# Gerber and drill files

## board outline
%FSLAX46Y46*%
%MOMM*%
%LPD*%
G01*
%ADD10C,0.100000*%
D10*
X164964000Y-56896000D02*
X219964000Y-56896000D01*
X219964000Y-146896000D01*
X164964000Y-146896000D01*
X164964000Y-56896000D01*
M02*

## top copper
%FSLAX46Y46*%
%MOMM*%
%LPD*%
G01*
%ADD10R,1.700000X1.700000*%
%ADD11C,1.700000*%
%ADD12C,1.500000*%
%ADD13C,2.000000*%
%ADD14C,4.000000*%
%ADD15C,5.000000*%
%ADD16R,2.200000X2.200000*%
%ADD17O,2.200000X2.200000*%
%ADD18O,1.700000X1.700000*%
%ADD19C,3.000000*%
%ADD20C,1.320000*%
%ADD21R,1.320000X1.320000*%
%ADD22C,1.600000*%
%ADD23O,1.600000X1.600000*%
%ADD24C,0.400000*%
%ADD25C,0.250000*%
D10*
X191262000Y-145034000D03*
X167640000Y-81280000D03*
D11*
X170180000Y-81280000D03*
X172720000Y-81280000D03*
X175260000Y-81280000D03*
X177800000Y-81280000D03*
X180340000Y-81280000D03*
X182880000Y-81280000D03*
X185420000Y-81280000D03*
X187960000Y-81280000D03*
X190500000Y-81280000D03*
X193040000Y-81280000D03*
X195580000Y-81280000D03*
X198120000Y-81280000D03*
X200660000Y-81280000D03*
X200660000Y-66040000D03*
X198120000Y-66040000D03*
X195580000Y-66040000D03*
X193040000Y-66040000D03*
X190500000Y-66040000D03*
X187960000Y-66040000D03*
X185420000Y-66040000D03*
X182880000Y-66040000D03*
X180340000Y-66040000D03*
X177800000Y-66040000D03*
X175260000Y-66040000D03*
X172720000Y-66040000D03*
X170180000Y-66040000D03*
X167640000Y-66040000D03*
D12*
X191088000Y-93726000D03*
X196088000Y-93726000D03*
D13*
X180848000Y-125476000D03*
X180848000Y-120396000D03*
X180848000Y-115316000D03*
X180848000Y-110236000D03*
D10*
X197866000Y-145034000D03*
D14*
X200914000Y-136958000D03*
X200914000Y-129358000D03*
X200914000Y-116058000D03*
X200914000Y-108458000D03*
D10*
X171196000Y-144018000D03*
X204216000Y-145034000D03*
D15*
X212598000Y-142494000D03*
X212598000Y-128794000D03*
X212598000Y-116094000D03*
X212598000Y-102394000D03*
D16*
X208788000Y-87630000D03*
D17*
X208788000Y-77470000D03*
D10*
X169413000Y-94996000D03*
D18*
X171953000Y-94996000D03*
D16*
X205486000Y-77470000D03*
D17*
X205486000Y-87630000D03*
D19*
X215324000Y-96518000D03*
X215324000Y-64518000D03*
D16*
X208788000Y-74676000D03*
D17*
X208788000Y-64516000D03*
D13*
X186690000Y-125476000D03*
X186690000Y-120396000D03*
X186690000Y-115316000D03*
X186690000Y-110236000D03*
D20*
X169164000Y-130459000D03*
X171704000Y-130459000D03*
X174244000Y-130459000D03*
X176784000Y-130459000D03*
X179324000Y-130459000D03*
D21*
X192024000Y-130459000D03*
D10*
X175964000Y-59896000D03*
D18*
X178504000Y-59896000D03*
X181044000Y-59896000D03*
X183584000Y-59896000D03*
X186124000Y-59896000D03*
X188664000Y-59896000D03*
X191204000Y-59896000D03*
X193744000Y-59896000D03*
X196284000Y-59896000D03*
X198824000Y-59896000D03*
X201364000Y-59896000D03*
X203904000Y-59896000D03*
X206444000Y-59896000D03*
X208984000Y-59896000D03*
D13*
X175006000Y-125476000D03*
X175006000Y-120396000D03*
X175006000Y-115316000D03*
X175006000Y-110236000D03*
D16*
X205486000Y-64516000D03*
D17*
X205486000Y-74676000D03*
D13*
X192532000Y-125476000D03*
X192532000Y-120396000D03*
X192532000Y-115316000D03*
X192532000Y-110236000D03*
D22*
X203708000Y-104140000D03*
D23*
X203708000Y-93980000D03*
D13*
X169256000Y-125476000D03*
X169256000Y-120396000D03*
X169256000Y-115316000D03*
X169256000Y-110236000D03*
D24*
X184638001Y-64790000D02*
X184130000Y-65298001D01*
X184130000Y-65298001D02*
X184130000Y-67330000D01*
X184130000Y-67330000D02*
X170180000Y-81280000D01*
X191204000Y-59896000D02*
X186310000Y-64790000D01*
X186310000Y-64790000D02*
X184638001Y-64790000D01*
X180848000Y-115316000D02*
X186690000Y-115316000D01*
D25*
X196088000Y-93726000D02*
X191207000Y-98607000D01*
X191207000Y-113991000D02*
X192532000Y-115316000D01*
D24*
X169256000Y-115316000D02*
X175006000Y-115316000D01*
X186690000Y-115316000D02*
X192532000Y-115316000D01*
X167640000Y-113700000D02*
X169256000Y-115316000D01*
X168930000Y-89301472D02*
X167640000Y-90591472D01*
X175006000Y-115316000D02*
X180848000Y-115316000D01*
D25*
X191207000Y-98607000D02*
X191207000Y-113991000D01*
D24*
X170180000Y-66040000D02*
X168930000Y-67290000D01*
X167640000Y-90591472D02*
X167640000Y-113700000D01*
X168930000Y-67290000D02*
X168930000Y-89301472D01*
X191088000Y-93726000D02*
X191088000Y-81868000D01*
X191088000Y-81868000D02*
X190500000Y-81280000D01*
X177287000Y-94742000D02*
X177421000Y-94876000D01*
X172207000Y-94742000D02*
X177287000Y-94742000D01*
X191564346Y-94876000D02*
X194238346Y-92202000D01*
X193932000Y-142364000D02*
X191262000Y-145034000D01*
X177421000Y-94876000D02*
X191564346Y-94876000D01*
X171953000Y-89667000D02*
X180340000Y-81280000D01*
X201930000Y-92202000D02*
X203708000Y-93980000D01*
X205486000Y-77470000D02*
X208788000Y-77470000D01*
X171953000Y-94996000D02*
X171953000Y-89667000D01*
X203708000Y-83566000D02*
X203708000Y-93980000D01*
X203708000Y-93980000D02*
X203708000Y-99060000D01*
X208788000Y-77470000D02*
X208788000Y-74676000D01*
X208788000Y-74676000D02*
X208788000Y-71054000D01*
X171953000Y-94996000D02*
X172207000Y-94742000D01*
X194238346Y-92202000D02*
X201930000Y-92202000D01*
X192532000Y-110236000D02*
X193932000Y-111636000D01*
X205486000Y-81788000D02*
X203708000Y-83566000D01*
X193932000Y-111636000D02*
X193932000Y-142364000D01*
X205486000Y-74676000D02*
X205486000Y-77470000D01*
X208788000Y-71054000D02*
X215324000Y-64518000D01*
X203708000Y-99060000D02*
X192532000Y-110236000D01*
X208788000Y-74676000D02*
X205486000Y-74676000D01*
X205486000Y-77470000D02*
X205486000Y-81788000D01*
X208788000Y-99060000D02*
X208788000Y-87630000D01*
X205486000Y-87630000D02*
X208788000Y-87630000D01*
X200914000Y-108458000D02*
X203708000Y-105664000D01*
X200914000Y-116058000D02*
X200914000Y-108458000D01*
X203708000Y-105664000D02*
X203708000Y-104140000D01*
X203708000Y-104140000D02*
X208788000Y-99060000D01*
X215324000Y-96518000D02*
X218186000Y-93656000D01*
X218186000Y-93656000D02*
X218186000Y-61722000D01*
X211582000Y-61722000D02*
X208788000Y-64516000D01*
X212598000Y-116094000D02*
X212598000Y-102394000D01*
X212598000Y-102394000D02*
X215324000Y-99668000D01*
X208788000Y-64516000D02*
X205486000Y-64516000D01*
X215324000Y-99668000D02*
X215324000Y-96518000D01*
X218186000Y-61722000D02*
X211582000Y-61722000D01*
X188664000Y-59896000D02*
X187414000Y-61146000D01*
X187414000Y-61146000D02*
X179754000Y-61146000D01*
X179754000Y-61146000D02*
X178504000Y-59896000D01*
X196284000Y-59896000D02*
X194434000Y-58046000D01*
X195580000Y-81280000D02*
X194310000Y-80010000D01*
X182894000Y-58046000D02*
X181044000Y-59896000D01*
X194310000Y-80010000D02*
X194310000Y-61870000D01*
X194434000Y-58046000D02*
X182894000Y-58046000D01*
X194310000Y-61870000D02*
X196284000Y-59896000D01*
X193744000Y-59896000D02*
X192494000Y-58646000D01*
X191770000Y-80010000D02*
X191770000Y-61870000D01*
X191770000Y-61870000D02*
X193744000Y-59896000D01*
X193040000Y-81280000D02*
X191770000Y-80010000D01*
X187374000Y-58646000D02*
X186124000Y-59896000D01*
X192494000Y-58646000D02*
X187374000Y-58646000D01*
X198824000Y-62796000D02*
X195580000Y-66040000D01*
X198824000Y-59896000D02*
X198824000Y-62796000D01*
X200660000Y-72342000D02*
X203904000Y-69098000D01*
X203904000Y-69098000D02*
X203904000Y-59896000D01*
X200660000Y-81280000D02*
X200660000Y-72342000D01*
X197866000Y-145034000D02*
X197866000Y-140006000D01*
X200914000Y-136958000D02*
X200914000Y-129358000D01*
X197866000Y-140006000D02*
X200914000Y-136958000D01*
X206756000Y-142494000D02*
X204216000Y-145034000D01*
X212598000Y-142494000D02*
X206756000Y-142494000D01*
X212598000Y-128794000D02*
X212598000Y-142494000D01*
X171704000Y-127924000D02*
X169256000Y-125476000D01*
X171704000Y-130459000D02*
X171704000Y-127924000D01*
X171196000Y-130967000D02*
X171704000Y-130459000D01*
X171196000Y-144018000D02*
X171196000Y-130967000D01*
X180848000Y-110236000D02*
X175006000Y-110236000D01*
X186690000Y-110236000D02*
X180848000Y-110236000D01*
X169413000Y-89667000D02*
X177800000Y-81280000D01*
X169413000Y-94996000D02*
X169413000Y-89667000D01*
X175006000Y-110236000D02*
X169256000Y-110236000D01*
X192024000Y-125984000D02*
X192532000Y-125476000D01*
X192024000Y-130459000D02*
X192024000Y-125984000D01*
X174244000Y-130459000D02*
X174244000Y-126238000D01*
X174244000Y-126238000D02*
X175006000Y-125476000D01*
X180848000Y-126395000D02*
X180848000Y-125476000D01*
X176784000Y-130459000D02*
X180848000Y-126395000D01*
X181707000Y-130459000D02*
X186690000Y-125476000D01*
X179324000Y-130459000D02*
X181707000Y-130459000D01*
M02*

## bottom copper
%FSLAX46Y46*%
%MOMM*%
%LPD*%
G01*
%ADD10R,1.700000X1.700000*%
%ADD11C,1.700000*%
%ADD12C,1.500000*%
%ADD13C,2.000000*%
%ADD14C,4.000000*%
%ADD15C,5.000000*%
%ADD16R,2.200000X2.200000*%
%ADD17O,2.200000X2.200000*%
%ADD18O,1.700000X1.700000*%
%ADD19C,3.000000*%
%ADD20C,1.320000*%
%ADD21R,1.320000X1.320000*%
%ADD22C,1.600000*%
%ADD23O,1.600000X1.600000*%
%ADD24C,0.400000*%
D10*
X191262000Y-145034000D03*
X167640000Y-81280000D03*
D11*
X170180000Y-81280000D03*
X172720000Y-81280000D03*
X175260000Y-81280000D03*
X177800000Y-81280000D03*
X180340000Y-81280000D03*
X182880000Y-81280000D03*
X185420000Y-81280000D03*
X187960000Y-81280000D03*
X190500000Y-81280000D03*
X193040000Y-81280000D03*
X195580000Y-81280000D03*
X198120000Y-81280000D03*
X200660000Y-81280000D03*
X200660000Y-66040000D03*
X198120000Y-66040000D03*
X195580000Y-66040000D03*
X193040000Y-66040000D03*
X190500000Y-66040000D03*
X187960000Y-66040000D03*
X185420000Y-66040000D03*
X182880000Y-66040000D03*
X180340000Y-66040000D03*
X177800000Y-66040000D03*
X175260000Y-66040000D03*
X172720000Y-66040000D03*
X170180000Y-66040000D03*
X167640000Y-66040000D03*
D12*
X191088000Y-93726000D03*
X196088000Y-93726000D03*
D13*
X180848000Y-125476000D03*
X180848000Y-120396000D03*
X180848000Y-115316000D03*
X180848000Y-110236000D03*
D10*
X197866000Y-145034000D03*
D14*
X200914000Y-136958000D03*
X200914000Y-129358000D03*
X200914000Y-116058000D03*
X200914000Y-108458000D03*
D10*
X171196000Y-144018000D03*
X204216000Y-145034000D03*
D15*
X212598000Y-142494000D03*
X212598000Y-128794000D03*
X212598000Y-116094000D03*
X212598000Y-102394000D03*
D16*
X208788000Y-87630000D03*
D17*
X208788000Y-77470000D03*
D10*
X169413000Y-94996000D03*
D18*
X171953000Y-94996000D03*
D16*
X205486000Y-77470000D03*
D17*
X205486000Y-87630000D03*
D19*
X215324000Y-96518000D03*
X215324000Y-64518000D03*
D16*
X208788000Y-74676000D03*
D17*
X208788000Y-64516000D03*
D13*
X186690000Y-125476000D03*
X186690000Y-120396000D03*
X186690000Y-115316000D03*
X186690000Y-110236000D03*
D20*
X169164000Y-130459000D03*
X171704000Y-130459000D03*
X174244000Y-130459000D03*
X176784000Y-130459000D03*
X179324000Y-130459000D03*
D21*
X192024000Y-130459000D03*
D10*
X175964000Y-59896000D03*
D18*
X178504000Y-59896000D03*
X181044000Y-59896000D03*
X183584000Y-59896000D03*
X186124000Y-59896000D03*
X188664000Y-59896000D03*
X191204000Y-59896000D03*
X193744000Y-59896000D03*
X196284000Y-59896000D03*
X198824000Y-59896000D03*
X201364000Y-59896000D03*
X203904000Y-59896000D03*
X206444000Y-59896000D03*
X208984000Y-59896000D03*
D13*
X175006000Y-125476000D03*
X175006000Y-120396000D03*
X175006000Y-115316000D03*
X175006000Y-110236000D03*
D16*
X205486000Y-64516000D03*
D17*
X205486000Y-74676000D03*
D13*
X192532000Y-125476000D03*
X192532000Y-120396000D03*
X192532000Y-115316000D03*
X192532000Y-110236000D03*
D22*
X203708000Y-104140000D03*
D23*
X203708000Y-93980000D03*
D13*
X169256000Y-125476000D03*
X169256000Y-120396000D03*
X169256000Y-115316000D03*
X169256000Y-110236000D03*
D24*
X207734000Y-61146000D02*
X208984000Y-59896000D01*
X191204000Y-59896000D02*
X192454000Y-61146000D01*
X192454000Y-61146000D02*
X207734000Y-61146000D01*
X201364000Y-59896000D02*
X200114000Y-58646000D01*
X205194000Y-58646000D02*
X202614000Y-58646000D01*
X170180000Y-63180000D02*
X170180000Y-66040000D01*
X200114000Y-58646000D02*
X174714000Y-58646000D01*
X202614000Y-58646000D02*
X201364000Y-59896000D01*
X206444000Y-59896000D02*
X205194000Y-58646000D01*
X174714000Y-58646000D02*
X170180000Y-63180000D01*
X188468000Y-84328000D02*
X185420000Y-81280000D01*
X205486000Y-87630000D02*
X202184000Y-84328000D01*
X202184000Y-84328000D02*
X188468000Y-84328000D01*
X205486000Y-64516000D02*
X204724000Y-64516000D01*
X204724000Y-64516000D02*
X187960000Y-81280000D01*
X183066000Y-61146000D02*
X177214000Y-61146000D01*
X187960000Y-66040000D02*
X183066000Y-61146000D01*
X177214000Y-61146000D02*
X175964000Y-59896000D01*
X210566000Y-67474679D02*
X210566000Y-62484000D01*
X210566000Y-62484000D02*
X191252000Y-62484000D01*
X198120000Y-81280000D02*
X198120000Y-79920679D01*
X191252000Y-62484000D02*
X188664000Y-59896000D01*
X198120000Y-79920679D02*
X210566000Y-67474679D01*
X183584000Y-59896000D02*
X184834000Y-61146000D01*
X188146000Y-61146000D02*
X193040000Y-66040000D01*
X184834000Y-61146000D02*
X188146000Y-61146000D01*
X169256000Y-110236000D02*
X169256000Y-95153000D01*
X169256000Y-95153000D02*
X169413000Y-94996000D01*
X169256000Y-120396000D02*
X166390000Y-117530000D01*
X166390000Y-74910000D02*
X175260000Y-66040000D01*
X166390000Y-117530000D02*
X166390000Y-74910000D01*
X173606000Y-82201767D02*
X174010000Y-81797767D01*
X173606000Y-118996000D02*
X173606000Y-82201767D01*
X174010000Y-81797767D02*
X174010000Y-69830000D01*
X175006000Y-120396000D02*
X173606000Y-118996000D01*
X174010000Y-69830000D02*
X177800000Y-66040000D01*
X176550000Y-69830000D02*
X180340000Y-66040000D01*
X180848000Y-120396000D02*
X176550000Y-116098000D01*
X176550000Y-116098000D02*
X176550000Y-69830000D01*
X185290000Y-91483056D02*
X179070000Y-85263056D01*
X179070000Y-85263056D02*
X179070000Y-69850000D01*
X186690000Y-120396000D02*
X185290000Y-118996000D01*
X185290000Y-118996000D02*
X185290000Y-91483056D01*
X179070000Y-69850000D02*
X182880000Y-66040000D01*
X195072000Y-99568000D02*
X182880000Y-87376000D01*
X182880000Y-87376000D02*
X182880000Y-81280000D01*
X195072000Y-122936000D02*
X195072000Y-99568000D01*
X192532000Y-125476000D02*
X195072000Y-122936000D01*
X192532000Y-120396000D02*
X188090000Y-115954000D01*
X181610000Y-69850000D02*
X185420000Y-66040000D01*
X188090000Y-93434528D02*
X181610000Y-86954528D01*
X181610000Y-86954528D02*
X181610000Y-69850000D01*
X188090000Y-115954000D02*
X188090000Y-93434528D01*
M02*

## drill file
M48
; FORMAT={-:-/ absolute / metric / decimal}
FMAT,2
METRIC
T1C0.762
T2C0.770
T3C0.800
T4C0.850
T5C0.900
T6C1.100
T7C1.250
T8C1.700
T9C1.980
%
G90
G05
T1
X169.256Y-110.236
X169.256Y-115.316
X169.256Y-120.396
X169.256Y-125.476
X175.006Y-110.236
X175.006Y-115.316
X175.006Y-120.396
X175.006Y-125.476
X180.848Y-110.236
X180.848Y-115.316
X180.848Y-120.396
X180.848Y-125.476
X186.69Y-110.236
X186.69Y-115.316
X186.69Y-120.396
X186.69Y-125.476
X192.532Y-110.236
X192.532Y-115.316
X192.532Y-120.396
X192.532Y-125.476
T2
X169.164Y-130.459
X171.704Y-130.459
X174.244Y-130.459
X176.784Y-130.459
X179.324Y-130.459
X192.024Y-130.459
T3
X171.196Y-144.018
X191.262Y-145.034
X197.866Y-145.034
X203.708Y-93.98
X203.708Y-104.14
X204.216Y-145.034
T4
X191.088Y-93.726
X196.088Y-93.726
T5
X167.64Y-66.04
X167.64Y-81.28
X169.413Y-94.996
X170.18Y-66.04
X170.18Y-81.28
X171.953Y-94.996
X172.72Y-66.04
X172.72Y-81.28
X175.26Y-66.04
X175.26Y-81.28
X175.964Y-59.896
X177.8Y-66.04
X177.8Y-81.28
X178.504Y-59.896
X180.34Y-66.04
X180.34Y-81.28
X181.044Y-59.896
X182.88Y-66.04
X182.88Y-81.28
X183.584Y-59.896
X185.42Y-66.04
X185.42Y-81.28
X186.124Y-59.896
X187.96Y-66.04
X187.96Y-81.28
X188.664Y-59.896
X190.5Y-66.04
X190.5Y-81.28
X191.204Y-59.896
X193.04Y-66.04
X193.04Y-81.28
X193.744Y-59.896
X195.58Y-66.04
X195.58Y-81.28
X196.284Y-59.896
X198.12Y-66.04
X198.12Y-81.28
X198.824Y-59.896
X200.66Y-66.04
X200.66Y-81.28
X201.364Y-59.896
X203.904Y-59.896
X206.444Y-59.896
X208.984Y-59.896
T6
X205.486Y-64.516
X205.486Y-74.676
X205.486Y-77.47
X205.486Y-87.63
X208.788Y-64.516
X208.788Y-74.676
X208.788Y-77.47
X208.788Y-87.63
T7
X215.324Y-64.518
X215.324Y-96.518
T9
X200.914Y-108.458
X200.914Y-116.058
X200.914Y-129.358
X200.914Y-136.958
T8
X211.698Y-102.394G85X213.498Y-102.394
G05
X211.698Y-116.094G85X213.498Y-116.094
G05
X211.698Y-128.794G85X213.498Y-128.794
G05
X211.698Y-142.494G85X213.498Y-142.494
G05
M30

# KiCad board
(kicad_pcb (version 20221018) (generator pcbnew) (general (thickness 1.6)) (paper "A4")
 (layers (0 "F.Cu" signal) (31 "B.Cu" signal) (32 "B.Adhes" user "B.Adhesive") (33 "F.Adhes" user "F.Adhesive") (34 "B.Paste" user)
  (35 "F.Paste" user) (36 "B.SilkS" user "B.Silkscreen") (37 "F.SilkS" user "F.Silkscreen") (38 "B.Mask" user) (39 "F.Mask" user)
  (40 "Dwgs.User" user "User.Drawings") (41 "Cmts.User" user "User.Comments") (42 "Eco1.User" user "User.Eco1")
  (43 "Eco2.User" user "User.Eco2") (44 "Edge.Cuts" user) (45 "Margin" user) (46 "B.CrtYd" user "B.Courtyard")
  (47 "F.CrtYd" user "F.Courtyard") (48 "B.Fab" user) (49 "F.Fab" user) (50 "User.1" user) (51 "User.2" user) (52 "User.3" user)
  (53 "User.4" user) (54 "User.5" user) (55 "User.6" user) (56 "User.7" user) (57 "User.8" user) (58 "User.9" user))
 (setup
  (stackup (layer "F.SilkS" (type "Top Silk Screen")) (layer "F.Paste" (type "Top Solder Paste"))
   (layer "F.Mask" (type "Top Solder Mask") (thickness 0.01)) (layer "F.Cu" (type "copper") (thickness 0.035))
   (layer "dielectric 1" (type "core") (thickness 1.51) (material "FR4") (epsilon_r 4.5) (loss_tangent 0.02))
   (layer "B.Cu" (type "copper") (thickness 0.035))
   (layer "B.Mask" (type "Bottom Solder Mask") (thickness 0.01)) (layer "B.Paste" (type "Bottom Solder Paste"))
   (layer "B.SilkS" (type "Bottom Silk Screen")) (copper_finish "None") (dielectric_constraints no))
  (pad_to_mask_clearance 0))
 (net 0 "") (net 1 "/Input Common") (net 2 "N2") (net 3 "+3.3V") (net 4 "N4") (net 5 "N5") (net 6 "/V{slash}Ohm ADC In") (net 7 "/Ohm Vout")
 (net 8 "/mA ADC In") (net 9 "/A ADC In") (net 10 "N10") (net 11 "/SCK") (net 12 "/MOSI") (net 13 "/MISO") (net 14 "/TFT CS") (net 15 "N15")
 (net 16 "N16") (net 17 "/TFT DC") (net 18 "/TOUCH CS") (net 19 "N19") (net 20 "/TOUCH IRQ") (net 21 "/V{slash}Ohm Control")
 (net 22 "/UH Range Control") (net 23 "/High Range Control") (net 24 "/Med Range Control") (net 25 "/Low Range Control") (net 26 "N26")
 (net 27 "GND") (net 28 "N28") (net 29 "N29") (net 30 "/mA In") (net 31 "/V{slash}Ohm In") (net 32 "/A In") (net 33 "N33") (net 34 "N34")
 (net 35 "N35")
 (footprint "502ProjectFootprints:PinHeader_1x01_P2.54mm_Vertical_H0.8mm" (layer "F.Cu") (at 191.262 145.034)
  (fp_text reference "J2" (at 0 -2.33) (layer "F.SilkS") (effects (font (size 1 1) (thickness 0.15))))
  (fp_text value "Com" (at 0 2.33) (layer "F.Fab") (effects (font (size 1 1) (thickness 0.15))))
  (pad "1" thru_hole rect (at 0 0) (size 1.7 1.7) (drill 0.8) (layers "*.Cu" "*.Mask") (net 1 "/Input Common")))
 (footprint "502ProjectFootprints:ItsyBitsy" (layer "F.Cu") (at 182.88 73.66 90)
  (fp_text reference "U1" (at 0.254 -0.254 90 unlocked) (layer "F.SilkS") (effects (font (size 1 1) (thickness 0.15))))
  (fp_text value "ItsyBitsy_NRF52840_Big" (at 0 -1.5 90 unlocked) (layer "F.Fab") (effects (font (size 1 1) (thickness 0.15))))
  (pad "1" thru_hole rect (at -7.62 -15.24 90) (size 1.7 1.7) (drill 0.9) (layers "*.Cu" "*.Mask") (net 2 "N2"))
  (pad "2" thru_hole circle (at -7.62 -12.7 90) (size 1.7 1.7) (drill 0.9) (layers "*.Cu" "*.Mask") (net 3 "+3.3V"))
  (pad "3" thru_hole circle (at -7.62 -10.16 90) (size 1.7 1.7) (drill 0.9) (layers "*.Cu" "*.Mask") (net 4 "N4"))
  (pad "4" thru_hole circle (at -7.62 -7.62 90) (size 1.7 1.7) (drill 0.9) (layers "*.Cu" "*.Mask") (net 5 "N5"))
  (pad "5" thru_hole circle (at -7.62 -5.08 90) (size 1.7 1.7) (drill 0.9) (layers "*.Cu" "*.Mask") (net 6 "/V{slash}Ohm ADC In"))
  (pad "6" thru_hole circle (at -7.62 -2.54 90) (size 1.7 1.7) (drill 0.9) (layers "*.Cu" "*.Mask") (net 1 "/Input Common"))
  (pad "7" thru_hole circle (at -7.62 0 90) (size 1.7 1.7) (drill 0.9) (layers "*.Cu" "*.Mask") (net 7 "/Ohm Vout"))
  (pad "8" thru_hole circle (at -7.62 2.54 90) (size 1.7 1.7) (drill 0.9) (layers "*.Cu" "*.Mask") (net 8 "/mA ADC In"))
  (pad "9" thru_hole circle (at -7.62 5.08 90) (size 1.7 1.7) (drill 0.9) (layers "*.Cu" "*.Mask") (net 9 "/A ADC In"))
  (pad "10" thru_hole circle (at -7.62 7.62 90) (size 1.7 1.7) (drill 0.9) (layers "*.Cu" "*.Mask") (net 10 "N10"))
  (pad "11" thru_hole circle (at -7.62 10.16 90) (size 1.7 1.7) (drill 0.9) (layers "*.Cu" "*.Mask") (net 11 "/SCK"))
  (pad "12" thru_hole circle (at -7.62 12.7 90) (size 1.7 1.7) (drill 0.9) (layers "*.Cu" "*.Mask") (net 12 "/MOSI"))
  (pad "13" thru_hole circle (at -7.62 15.24 90) (size 1.7 1.7) (drill 0.9) (layers "*.Cu" "*.Mask") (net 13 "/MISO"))
  (pad "14" thru_hole circle (at -7.62 17.78 90) (size 1.7 1.7) (drill 0.9) (layers "*.Cu" "*.Mask") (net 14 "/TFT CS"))
  (pad "15" thru_hole circle (at 7.62 17.78 90) (size 1.7 1.7) (drill 0.9) (layers "*.Cu" "*.Mask") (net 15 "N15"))
  (pad "16" thru_hole circle (at 7.62 15.24 90) (size 1.7 1.7) (drill 0.9) (layers "*.Cu" "*.Mask") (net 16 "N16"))
  (pad "17" thru_hole circle (at 7.62 12.7 90) (size 1.7 1.7) (drill 0.9) (layers "*.Cu" "*.Mask") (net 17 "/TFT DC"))
  (pad "18" thru_hole circle (at 7.62 10.16 90) (size 1.7 1.7) (drill 0.9) (layers "*.Cu" "*.Mask") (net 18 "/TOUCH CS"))
  (pad "19" thru_hole circle (at 7.62 7.62 90) (size 1.7 1.7) (drill 0.9) (layers "*.Cu" "*.Mask") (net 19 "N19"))
  (pad "20" thru_hole circle (at 7.62 5.08 90) (size 1.7 1.7) (drill 0.9) (layers "*.Cu" "*.Mask") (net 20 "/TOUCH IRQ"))
  (pad "21" thru_hole circle (at 7.62 2.54 90) (size 1.7 1.7) (drill 0.9) (layers "*.Cu" "*.Mask") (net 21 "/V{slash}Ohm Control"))
  (pad "22" thru_hole circle (at 7.62 0 90) (size 1.7 1.7) (drill 0.9) (layers "*.Cu" "*.Mask") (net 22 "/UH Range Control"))
  (pad "23" thru_hole circle (at 7.62 -2.54 90) (size 1.7 1.7) (drill 0.9) (layers "*.Cu" "*.Mask") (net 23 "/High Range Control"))
  (pad "24" thru_hole circle (at 7.62 -5.08 90) (size 1.7 1.7) (drill 0.9) (layers "*.Cu" "*.Mask") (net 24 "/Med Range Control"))
  (pad "25" thru_hole circle (at 7.62 -7.62 90) (size 1.7 1.7) (drill 0.9) (layers "*.Cu" "*.Mask") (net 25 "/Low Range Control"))
  (pad "26" thru_hole circle (at 7.62 -10.16 90) (size 1.7 1.7) (drill 0.9) (layers "*.Cu" "*.Mask") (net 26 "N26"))
  (pad "27" thru_hole circle (at 7.62 -12.7 90) (size 1.7 1.7) (drill 0.9) (layers "*.Cu" "*.Mask") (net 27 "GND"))
  (pad "28" thru_hole circle (at 7.62 -15.24 90) (size 1.7 1.7) (drill 0.9) (layers "*.Cu" "*.Mask") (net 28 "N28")))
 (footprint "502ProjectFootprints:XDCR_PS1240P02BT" (layer "F.Cu") (at 193.588 93.726)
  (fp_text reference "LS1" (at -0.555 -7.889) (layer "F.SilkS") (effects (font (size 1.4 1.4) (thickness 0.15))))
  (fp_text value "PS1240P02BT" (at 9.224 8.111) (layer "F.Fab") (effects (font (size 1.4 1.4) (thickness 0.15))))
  (pad "1" thru_hole circle (at -2.5 0) (size 1.5 1.5) (drill 0.85) (layers "*.Cu" "*.Mask") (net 10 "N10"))
  (pad "2" thru_hole circle (at 2.5 0) (size 1.5 1.5) (drill 0.85) (layers "*.Cu" "*.Mask") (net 27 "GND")))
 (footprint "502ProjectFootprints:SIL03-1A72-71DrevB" (layer "F.Cu") (at 180.848 117.856 90)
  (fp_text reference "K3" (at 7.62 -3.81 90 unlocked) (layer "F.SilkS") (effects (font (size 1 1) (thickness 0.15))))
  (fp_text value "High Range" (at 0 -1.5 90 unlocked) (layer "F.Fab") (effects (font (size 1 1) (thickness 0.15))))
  (pad "1" thru_hole circle (at -7.62 0 90) (size 2 2) (drill 0.762) (layers "*.Cu" "*.Mask") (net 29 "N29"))
  (pad "3" thru_hole circle (at -2.54 0 90) (size 2 2) (drill 0.762) (layers "*.Cu" "*.Mask") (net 23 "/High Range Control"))
  (pad "5" thru_hole circle (at 2.54 0 90) (size 2 2) (drill 0.762) (layers "*.Cu" "*.Mask") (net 27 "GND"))
  (pad "7" thru_hole circle (at 7.62 0 90) (size 2 2) (drill 0.762) (layers "*.Cu" "*.Mask") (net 6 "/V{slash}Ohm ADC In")))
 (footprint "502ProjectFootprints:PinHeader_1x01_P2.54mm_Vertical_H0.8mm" (layer "F.Cu") (at 197.866 145.034)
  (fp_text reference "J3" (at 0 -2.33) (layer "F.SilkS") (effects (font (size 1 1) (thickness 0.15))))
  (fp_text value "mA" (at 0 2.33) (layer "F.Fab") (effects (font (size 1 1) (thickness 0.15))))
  (pad "1" thru_hole rect (at 0 0) (size 1.7 1.7) (drill 0.8) (layers "*.Cu" "*.Mask") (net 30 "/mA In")))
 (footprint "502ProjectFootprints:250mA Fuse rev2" (layer "F.Cu") (at 200.914 122.708 90)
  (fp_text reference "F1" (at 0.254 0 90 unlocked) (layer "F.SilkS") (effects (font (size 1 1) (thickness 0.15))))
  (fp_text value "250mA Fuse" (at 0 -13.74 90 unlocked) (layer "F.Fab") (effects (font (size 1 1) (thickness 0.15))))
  (pad "1" thru_hole circle (at -14.25 0 90) (size 4 4) (drill 1.98) (layers "*.Cu" "*.Mask") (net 30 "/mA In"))
  (pad "2" thru_hole circle (at -6.65 0 90) (size 4 4) (drill 1.98) (layers "*.Cu" "*.Mask") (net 30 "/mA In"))
  (pad "3" thru_hole circle (at 6.65 0 90) (size 4 4) (drill 1.98) (layers "*.Cu" "*.Mask") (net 8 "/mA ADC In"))
  (pad "4" thru_hole circle (at 14.25 0 90) (size 4 4) (drill 1.98) (layers "*.Cu" "*.Mask") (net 8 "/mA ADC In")))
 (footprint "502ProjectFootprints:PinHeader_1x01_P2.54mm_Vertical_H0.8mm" (layer "F.Cu") (at 171.196 144.018)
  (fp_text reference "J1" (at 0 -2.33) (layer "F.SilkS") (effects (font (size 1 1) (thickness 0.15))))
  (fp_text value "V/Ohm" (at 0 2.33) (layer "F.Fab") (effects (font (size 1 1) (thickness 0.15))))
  (pad "1" thru_hole rect (at 0 0) (size 1.7 1.7) (drill 0.8) (layers "*.Cu" "*.Mask") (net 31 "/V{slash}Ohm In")))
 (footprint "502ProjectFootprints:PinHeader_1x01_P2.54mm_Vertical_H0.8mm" (layer "F.Cu") (at 204.216 145.034)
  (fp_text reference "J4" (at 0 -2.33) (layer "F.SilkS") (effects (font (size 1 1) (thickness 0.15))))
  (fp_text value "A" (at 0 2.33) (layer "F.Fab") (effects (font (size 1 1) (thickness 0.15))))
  (pad "1" thru_hole rect (at 0 0) (size 1.7 1.7) (drill 0.8) (layers "*.Cu" "*.Mask") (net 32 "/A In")))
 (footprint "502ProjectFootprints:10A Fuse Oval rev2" (layer "F.Cu") (at 212.598 122.444 90)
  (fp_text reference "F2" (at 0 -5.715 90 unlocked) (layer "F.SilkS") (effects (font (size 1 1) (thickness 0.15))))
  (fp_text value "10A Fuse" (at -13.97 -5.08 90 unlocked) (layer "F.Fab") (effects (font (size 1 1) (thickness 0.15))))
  (pad "1" thru_hole circle (at -20.05 0 90) (size 5 5) (drill oval 1.7 3.5) (layers "*.Cu" "*.Mask") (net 32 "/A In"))
  (pad "2" thru_hole circle (at -6.35 0 90) (size 5 5) (drill oval 1.7 3.5) (layers "*.Cu" "*.Mask") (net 32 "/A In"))
  (pad "3" thru_hole circle (at 6.35 0 90) (size 5 5) (drill oval 1.7 3.5) (layers "*.Cu" "*.Mask") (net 9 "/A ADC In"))
  (pad "4" thru_hole circle (at 20.05 0 90) (size 5 5) (drill oval 1.7 3.5) (layers "*.Cu" "*.Mask") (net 9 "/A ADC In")))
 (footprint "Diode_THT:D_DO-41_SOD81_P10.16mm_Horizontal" (layer "F.Cu") (at 208.788 87.63 90)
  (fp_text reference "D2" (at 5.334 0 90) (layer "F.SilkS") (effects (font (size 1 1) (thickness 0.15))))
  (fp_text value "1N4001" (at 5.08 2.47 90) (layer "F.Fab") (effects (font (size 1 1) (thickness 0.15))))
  (pad "1" thru_hole rect (at 0 0 90) (size 2.2 2.2) (drill 1.1) (layers "*.Cu" "*.Mask") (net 8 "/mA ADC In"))
  (pad "2" thru_hole oval (at 10.16 0 90) (size 2.2 2.2) (drill 1.1) (layers "*.Cu" "*.Mask") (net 1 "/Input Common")))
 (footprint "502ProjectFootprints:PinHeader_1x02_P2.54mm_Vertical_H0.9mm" (layer "F.Cu") (at 169.413 94.996 90)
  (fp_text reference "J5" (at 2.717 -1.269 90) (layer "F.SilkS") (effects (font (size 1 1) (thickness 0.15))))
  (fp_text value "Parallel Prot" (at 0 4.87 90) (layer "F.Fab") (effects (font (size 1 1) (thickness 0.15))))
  (pad "1" thru_hole rect (at 0 0 90) (size 1.7 1.7) (drill 0.9) (layers "*.Cu" "*.Mask") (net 6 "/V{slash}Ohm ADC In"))
  (pad "2" thru_hole oval (at 0 2.54 90) (size 1.7 1.7) (drill 0.9) (layers "*.Cu" "*.Mask") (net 1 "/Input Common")))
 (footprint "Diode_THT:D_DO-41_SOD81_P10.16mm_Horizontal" (layer "F.Cu") (at 205.486 77.47 -90)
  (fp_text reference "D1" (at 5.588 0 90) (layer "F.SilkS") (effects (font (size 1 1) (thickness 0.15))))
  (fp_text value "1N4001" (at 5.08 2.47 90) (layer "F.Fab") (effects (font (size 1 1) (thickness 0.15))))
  (pad "1" thru_hole rect (at 0 0 270) (size 2.2 2.2) (drill 1.1) (layers "*.Cu" "*.Mask") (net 1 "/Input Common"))
  (pad "2" thru_hole oval (at 10.16 0 270) (size 2.2 2.2) (drill 1.1) (layers "*.Cu" "*.Mask") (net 8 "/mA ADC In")))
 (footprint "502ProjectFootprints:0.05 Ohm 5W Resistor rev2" (layer "F.Cu") (at 211.074 70.358 90)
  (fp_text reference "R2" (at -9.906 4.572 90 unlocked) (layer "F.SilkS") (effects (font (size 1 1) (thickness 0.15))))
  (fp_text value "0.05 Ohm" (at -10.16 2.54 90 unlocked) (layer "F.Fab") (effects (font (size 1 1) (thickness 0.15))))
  (pad "1" thru_hole circle (at -26.16 4.25 90) (size 3 3) (drill 1.25) (layers "*.Cu" "*.Mask") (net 9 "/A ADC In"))
  (pad "2" thru_hole circle (at 5.84 4.25 90) (size 3 3) (drill 1.25) (layers "*.Cu" "*.Mask") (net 1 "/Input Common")))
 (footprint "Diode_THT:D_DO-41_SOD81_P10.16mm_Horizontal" (layer "F.Cu") (at 208.788 74.676 90)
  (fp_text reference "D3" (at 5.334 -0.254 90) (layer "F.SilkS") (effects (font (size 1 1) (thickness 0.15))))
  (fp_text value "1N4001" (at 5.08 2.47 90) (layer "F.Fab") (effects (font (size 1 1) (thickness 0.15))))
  (pad "1" thru_hole rect (at 0 0 90) (size 2.2 2.2) (drill 1.1) (layers "*.Cu" "*.Mask") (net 1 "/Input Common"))
  (pad "2" thru_hole oval (at 10.16 0 90) (size 2.2 2.2) (drill 1.1) (layers "*.Cu" "*.Mask") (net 9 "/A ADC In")))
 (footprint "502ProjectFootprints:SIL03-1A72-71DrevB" (layer "F.Cu") (at 186.69 117.856 90)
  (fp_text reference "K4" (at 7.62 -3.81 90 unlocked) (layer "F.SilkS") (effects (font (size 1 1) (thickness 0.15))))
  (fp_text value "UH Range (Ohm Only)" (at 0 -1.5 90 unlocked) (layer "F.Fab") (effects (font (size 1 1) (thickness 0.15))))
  (pad "1" thru_hole circle (at -7.62 0 90) (size 2 2) (drill 0.762) (layers "*.Cu" "*.Mask") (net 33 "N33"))
  (pad "3" thru_hole circle (at -2.54 0 90) (size 2 2) (drill 0.762) (layers "*.Cu" "*.Mask") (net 22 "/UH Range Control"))
  (pad "5" thru_hole circle (at 2.54 0 90) (size 2 2) (drill 0.762) (layers "*.Cu" "*.Mask") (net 27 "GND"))
  (pad "7" thru_hole circle (at 7.62 0 90) (size 2 2) (drill 0.762) (layers "*.Cu" "*.Mask") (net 6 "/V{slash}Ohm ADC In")))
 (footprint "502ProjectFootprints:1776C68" (layer "F.Cu") (at 192.024 130.459 180)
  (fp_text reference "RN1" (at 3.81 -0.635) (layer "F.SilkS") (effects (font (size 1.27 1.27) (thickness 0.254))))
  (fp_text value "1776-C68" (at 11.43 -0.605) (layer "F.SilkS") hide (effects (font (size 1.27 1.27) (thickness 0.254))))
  (pad "1" thru_hole circle (at 22.86 0 180) (size 1.32 1.32) (drill 0.77) (layers "*.Cu" "*.Mask") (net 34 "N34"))
  (pad "2" thru_hole circle (at 20.32 0 180) (size 1.32 1.32) (drill 0.77) (layers "*.Cu" "*.Mask") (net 31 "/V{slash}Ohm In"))
  (pad "3" thru_hole circle (at 17.78 0 180) (size 1.32 1.32) (drill 0.77) (layers "*.Cu" "*.Mask") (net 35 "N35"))
  (pad "4" thru_hole circle (at 15.24 0 180) (size 1.32 1.32) (drill 0.77) (layers "*.Cu" "*.Mask") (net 29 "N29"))
  (pad "5" thru_hole circle (at 12.7 0 180) (size 1.32 1.32) (drill 0.77) (layers "*.Cu" "*.Mask") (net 33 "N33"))
  (pad "6" thru_hole rect (at 0 0 180) (size 1.32 1.32) (drill 0.77) (layers "*.Cu" "*.Mask") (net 7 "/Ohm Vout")))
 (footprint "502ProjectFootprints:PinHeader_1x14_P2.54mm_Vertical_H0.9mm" (layer "F.Cu") (at 175.964 59.896 90)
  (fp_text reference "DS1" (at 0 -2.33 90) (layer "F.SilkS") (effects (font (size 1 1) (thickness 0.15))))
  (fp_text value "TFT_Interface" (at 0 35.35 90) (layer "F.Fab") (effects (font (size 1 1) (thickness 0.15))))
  (pad "1" thru_hole rect (at 0 0 90) (size 1.7 1.7) (drill 0.9) (layers "*.Cu" "*.Mask") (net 20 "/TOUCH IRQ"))
  (pad "2" thru_hole oval (at 0 2.54 90) (size 1.7 1.7) (drill 0.9) (layers "*.Cu" "*.Mask") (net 13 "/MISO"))
  (pad "3" thru_hole oval (at 0 5.08 90) (size 1.7 1.7) (drill 0.9) (layers "*.Cu" "*.Mask") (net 12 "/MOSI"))
  (pad "4" thru_hole oval (at 0 7.62 90) (size 1.7 1.7) (drill 0.9) (layers "*.Cu" "*.Mask") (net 18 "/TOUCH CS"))
  (pad "5" thru_hole oval (at 0 10.16 90) (size 1.7 1.7) (drill 0.9) (layers "*.Cu" "*.Mask") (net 11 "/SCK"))
  (pad "6" thru_hole oval (at 0 12.7 90) (size 1.7 1.7) (drill 0.9) (layers "*.Cu" "*.Mask") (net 13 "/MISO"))
  (pad "7" thru_hole oval (at 0 15.24 90) (size 1.7 1.7) (drill 0.9) (layers "*.Cu" "*.Mask") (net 3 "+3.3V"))
  (pad "8" thru_hole oval (at 0 17.78 90) (size 1.7 1.7) (drill 0.9) (layers "*.Cu" "*.Mask") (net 11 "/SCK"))
  (pad "9" thru_hole oval (at 0 20.32 90) (size 1.7 1.7) (drill 0.9) (layers "*.Cu" "*.Mask") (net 12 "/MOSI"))
  (pad "10" thru_hole oval (at 0 22.86 90) (size 1.7 1.7) (drill 0.9) (layers "*.Cu" "*.Mask") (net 17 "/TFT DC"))
  (pad "11" thru_hole oval (at 0 25.4 90) (size 1.7 1.7) (drill 0.9) (layers "*.Cu" "*.Mask") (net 27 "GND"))
  (pad "12" thru_hole oval (at 0 27.94 90) (size 1.7 1.7) (drill 0.9) (layers "*.Cu" "*.Mask") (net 14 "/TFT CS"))
  (pad "13" thru_hole oval (at 0 30.48 90) (size 1.7 1.7) (drill 0.9) (layers "*.Cu" "*.Mask") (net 27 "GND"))
  (pad "14" thru_hole oval (at 0 33.02 90) (size 1.7 1.7) (drill 0.9) (layers "*.Cu" "*.Mask") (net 3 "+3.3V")))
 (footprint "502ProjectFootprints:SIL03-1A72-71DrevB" (layer "F.Cu") (at 175.006 117.856 90)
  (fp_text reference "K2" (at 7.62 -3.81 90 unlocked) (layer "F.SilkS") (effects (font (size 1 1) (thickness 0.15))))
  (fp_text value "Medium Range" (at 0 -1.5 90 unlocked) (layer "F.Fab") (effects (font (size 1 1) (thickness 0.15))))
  (pad "1" thru_hole circle (at -7.62 0 90) (size 2 2) (drill 0.762) (layers "*.Cu" "*.Mask") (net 35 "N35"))
  (pad "3" thru_hole circle (at -2.54 0 90) (size 2 2) (drill 0.762) (layers "*.Cu" "*.Mask") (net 24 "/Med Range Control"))
  (pad "5" thru_hole circle (at 2.54 0 90) (size 2 2) (drill 0.762) (layers "*.Cu" "*.Mask") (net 27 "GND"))
  (pad "7" thru_hole circle (at 7.62 0 90) (size 2 2) (drill 0.762) (layers "*.Cu" "*.Mask") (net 6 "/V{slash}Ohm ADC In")))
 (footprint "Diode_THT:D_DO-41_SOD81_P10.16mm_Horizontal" (layer "F.Cu") (at 205.486 64.516 -90)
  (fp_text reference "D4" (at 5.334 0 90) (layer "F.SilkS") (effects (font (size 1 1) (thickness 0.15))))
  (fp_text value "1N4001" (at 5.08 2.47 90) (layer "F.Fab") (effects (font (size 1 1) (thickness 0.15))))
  (pad "1" thru_hole rect (at 0 0 270) (size 2.2 2.2) (drill 1.1) (layers "*.Cu" "*.Mask") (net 9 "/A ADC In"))
  (pad "2" thru_hole oval (at 10.16 0 270) (size 2.2 2.2) (drill 1.1) (layers "*.Cu" "*.Mask") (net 1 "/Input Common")))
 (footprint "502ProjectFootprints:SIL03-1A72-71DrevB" (layer "F.Cu") (at 192.532 117.856 90)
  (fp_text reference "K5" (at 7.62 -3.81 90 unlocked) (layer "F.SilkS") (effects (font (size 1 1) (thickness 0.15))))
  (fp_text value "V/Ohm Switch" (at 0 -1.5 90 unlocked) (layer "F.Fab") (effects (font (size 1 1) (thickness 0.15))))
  (pad "1" thru_hole circle (at -7.62 0 90) (size 2 2) (drill 0.762) (layers "*.Cu" "*.Mask") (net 7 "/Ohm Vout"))
  (pad "3" thru_hole circle (at -2.54 0 90) (size 2 2) (drill 0.762) (layers "*.Cu" "*.Mask") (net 21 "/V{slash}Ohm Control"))
  (pad "5" thru_hole circle (at 2.54 0 90) (size 2 2) (drill 0.762) (layers "*.Cu" "*.Mask") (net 27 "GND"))
  (pad "7" thru_hole circle (at 7.62 0 90) (size 2 2) (drill 0.762) (layers "*.Cu" "*.Mask") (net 1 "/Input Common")))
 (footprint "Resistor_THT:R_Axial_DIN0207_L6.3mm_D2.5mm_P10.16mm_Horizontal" (layer "F.Cu") (at 203.708 104.14 90)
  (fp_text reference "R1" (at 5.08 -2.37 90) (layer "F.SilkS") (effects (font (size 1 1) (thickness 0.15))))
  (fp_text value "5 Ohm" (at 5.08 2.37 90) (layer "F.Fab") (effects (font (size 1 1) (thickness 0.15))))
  (pad "1" thru_hole circle (at 0 0 90) (size 1.6 1.6) (drill 0.8) (layers "*.Cu" "*.Mask") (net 8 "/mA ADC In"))
  (pad "2" thru_hole oval (at 10.16 0 90) (size 1.6 1.6) (drill 0.8) (layers "*.Cu" "*.Mask") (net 1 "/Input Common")))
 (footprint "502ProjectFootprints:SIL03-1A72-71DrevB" (layer "F.Cu") (at 169.256 117.856 90)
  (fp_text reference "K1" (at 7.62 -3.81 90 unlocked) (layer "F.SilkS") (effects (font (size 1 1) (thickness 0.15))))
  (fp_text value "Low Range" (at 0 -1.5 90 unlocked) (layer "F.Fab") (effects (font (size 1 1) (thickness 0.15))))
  (pad "1" thru_hole circle (at -7.62 0 90) (size 2 2) (drill 0.762) (layers "*.Cu" "*.Mask") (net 31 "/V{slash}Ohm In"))
  (pad "3" thru_hole circle (at -2.54 0 90) (size 2 2) (drill 0.762) (layers "*.Cu" "*.Mask") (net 25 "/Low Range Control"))
  (pad "5" thru_hole circle (at 2.54 0 90) (size 2 2) (drill 0.762) (layers "*.Cu" "*.Mask") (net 27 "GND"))
  (pad "7" thru_hole circle (at 7.62 0 90) (size 2 2) (drill 0.762) (layers "*.Cu" "*.Mask") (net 6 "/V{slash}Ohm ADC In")))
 (gr_rect (start 164.964 56.896) (end 219.964 146.896) (stroke (width 0.1) (type default)) (fill none) (layer "Edge.Cuts"))
 (segment (start 184.638001 64.79) (end 184.13 65.298001) (width 0.4) (layer "F.Cu") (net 3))
 (segment (start 184.13 65.298001) (end 184.13 67.33) (width 0.4) (layer "F.Cu") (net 3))
 (segment (start 184.13 67.33) (end 170.18 81.28) (width 0.4) (layer "F.Cu") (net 3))
 (segment (start 191.204 59.896) (end 186.31 64.79) (width 0.4) (layer "F.Cu") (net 3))
 (segment (start 186.31 64.79) (end 184.638001 64.79) (width 0.4) (layer "F.Cu") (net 3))
 (segment (start 207.734 61.146) (end 208.984 59.896) (width 0.4) (layer "B.Cu") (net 3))
 (segment (start 191.204 59.896) (end 192.454 61.146) (width 0.4) (layer "B.Cu") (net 3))
 (segment (start 192.454 61.146) (end 207.734 61.146) (width 0.4) (layer "B.Cu") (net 3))
 (segment (start 180.848 115.316) (end 186.69 115.316) (width 0.4) (layer "F.Cu") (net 27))
 (segment (start 196.088 93.726) (end 191.207 98.607) (width 0.25) (layer "F.Cu") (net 27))
 (segment (start 191.207 113.991) (end 192.532 115.316) (width 0.25) (layer "F.Cu") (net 27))
 (segment (start 169.256 115.316) (end 175.006 115.316) (width 0.4) (layer "F.Cu") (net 27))
 (segment (start 186.69 115.316) (end 192.532 115.316) (width 0.4) (layer "F.Cu") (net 27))
 (segment (start 167.64 113.7) (end 169.256 115.316) (width 0.4) (layer "F.Cu") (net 27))
 (segment (start 168.93 89.301472) (end 167.64 90.591472) (width 0.4) (layer "F.Cu") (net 27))
 (segment (start 175.006 115.316) (end 180.848 115.316) (width 0.4) (layer "F.Cu") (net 27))
 (segment (start 191.207 98.607) (end 191.207 113.991) (width 0.25) (layer "F.Cu") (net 27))
 (segment (start 170.18 66.04) (end 168.93 67.29) (width 0.4) (layer "F.Cu") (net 27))
 (segment (start 167.64 90.591472) (end 167.64 113.7) (width 0.4) (layer "F.Cu") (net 27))
 (segment (start 168.93 67.29) (end 168.93 89.301472) (width 0.4) (layer "F.Cu") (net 27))
 (segment (start 201.364 59.896) (end 200.114 58.646) (width 0.4) (layer "B.Cu") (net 27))
 (segment (start 205.194 58.646) (end 202.614 58.646) (width 0.4) (layer "B.Cu") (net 27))
 (segment (start 170.18 63.18) (end 170.18 66.04) (width 0.4) (layer "B.Cu") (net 27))
 (segment (start 200.114 58.646) (end 174.714 58.646) (width 0.4) (layer "B.Cu") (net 27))
 (segment (start 202.614 58.646) (end 201.364 59.896) (width 0.4) (layer "B.Cu") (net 27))
 (segment (start 206.444 59.896) (end 205.194 58.646) (width 0.4) (layer "B.Cu") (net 27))
 (segment (start 174.714 58.646) (end 170.18 63.18) (width 0.4) (layer "B.Cu") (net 27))
 (segment (start 191.088 93.726) (end 191.088 81.868) (width 0.4) (layer "F.Cu") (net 10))
 (segment (start 191.088 81.868) (end 190.5 81.28) (width 0.4) (layer "F.Cu") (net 10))
 (segment (start 177.287 94.742) (end 177.421 94.876) (width 0.4) (layer "F.Cu") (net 1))
 (segment (start 172.207 94.742) (end 177.287 94.742) (width 0.4) (layer "F.Cu") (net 1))
 (segment (start 191.564346 94.876) (end 194.238346 92.202) (width 0.4) (layer "F.Cu") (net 1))
 (segment (start 193.932 142.364) (end 191.262 145.034) (width 0.4) (layer "F.Cu") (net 1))
 (segment (start 177.421 94.876) (end 191.564346 94.876) (width 0.4) (layer "F.Cu") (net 1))
 (segment (start 171.953 89.667) (end 180.34 81.28) (width 0.4) (layer "F.Cu") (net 1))
 (segment (start 201.93 92.202) (end 203.708 93.98) (width 0.4) (layer "F.Cu") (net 1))
 (segment (start 205.486 77.47) (end 208.788 77.47) (width 0.4) (layer "F.Cu") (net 1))
 (segment (start 171.953 94.996) (end 171.953 89.667) (width 0.4) (layer "F.Cu") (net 1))
 (segment (start 203.708 83.566) (end 203.708 93.98) (width 0.4) (layer "F.Cu") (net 1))
 (segment (start 203.708 93.98) (end 203.708 99.06) (width 0.4) (layer "F.Cu") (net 1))
 (segment (start 208.788 77.47) (end 208.788 74.676) (width 0.4) (layer "F.Cu") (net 1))
 (segment (start 208.788 74.676) (end 208.788 71.054) (width 0.4) (layer "F.Cu") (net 1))
 (segment (start 171.953 94.996) (end 172.207 94.742) (width 0.4) (layer "F.Cu") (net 1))
 (segment (start 194.238346 92.202) (end 201.93 92.202) (width 0.4) (layer "F.Cu") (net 1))
 (segment (start 192.532 110.236) (end 193.932 111.636) (width 0.4) (layer "F.Cu") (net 1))
 (segment (start 205.486 81.788) (end 203.708 83.566) (width 0.4) (layer "F.Cu") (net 1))
 (segment (start 193.932 111.636) (end 193.932 142.364) (width 0.4) (layer "F.Cu") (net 1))
 (segment (start 205.486 74.676) (end 205.486 77.47) (width 0.4) (layer "F.Cu") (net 1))
 (segment (start 208.788 71.054) (end 215.324 64.518) (width 0.4) (layer "F.Cu") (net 1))
 (segment (start 203.708 99.06) (end 192.532 110.236) (width 0.4) (layer "F.Cu") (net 1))
 (segment (start 208.788 74.676) (end 205.486 74.676) (width 0.4) (layer "F.Cu") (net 1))
 (segment (start 205.486 77.47) (end 205.486 81.788) (width 0.4) (layer "F.Cu") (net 1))
 (segment (start 208.788 99.06) (end 208.788 87.63) (width 0.4) (layer "F.Cu") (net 8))
 (segment (start 205.486 87.63) (end 208.788 87.63) (width 0.4) (layer "F.Cu") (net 8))
 (segment (start 200.914 108.458) (end 203.708 105.664) (width 0.4) (layer "F.Cu") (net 8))
 (segment (start 200.914 116.058) (end 200.914 108.458) (width 0.4) (layer "F.Cu") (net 8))
 (segment (start 203.708 105.664) (end 203.708 104.14) (width 0.4) (layer "F.Cu") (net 8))
 (segment (start 203.708 104.14) (end 208.788 99.06) (width 0.4) (layer "F.Cu") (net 8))
 (segment (start 188.468 84.328) (end 185.42 81.28) (width 0.4) (layer "B.Cu") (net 8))
 (segment (start 205.486 87.63) (end 202.184 84.328) (width 0.4) (layer "B.Cu") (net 8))
 (segment (start 202.184 84.328) (end 188.468 84.328) (width 0.4) (layer "B.Cu") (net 8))
 (segment (start 215.324 96.518) (end 218.186 93.656) (width 0.4) (layer "F.Cu") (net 9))
 (segment (start 218.186 93.656) (end 218.186 61.722) (width 0.4) (layer "F.Cu") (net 9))
 (segment (start 211.582 61.722) (end 208.788 64.516) (width 0.4) (layer "F.Cu") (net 9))
 (segment (start 212.598 116.094) (end 212.598 102.394) (width 0.4) (layer "F.Cu") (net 9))
 (segment (start 212.598 102.394) (end 215.324 99.668) (width 0.4) (layer "F.Cu") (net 9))
 (segment (start 208.788 64.516) (end 205.486 64.516) (width 0.4) (layer "F.Cu") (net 9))
 (segment (start 215.324 99.668) (end 215.324 96.518) (width 0.4) (layer "F.Cu") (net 9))
 (segment (start 218.186 61.722) (end 211.582 61.722) (width 0.4) (layer "F.Cu") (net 9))
 (segment (start 205.486 64.516) (end 204.724 64.516) (width 0.4) (layer "B.Cu") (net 9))
 (segment (start 204.724 64.516) (end 187.96 81.28) (width 0.4) (layer "B.Cu") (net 9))
 (segment (start 183.066 61.146) (end 177.214 61.146) (width 0.4) (layer "B.Cu") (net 20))
 (segment (start 187.96 66.04) (end 183.066 61.146) (width 0.4) (layer "B.Cu") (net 20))
 (segment (start 177.214 61.146) (end 175.964 59.896) (width 0.4) (layer "B.Cu") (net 20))
 (segment (start 188.664 59.896) (end 187.414 61.146) (width 0.4) (layer "F.Cu") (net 13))
 (segment (start 187.414 61.146) (end 179.754 61.146) (width 0.4) (layer "F.Cu") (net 13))
 (segment (start 179.754 61.146) (end 178.504 59.896) (width 0.4) (layer "F.Cu") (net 13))
 (segment (start 210.566 67.474679) (end 210.566 62.484) (width 0.4) (layer "B.Cu") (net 13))
 (segment (start 210.566 62.484) (end 191.252 62.484) (width 0.4) (layer "B.Cu") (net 13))
 (segment (start 198.12 81.28) (end 198.12 79.920679) (width 0.4) (layer "B.Cu") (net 13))
 (segment (start 191.252 62.484) (end 188.664 59.896) (width 0.4) (layer "B.Cu") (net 13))
 (segment (start 198.12 79.920679) (end 210.566 67.474679) (width 0.4) (layer "B.Cu") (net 13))
 (segment (start 196.284 59.896) (end 194.434 58.046) (width 0.4) (layer "F.Cu") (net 12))
 (segment (start 195.58 81.28) (end 194.31 80.01) (width 0.4) (layer "F.Cu") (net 12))
 (segment (start 182.894 58.046) (end 181.044 59.896) (width 0.4) (layer "F.Cu") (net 12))
 (segment (start 194.31 80.01) (end 194.31 61.87) (width 0.4) (layer "F.Cu") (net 12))
 (segment (start 194.434 58.046) (end 182.894 58.046) (width 0.4) (layer "F.Cu") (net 12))
 (segment (start 194.31 61.87) (end 196.284 59.896) (width 0.4) (layer "F.Cu") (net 12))
 (segment (start 183.584 59.896) (end 184.834 61.146) (width 0.4) (layer "B.Cu") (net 18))
 (segment (start 188.146 61.146) (end 193.04 66.04) (width 0.4) (layer "B.Cu") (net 18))
 (segment (start 184.834 61.146) (end 188.146 61.146) (width 0.4) (layer "B.Cu") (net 18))
 (segment (start 193.744 59.896) (end 192.494 58.646) (width 0.4) (layer "F.Cu") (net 11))
 (segment (start 191.77 80.01) (end 191.77 61.87) (width 0.4) (layer "F.Cu") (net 11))
 (segment (start 191.77 61.87) (end 193.744 59.896) (width 0.4) (layer "F.Cu") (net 11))
 (segment (start 193.04 81.28) (end 191.77 80.01) (width 0.4) (layer "F.Cu") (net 11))
 (segment (start 187.374 58.646) (end 186.124 59.896) (width 0.4) (layer "F.Cu") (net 11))
 (segment (start 192.494 58.646) (end 187.374 58.646) (width 0.4) (layer "F.Cu") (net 11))
 (segment (start 198.824 62.796) (end 195.58 66.04) (width 0.4) (layer "F.Cu") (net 17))
 (segment (start 198.824 59.896) (end 198.824 62.796) (width 0.4) (layer "F.Cu") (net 17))
 (segment (start 200.66 72.342) (end 203.904 69.098) (width 0.4) (layer "F.Cu") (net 14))
 (segment (start 203.904 69.098) (end 203.904 59.896) (width 0.4) (layer "F.Cu") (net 14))
 (segment (start 200.66 81.28) (end 200.66 72.342) (width 0.4) (layer "F.Cu") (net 14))
 (segment (start 197.866 145.034) (end 197.866 140.006) (width 0.4) (layer "F.Cu") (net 30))
 (segment (start 200.914 136.958) (end 200.914 129.358) (width 0.4) (layer "F.Cu") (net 30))
 (segment (start 197.866 140.006) (end 200.914 136.958) (width 0.4) (layer "F.Cu") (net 30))
 (segment (start 206.756 142.494) (end 204.216 145.034) (width 0.4) (layer "F.Cu") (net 32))
 (segment (start 212.598 142.494) (end 206.756 142.494) (width 0.4) (layer "F.Cu") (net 32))
 (segment (start 212.598 128.794) (end 212.598 142.494) (width 0.4) (layer "F.Cu") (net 32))
 (segment (start 171.704 127.924) (end 169.256 125.476) (width 0.4) (layer "F.Cu") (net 31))
 (segment (start 171.704 130.459) (end 171.704 127.924) (width 0.4) (layer "F.Cu") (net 31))
 (segment (start 171.196 130.967) (end 171.704 130.459) (width 0.4) (layer "F.Cu") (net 31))
 (segment (start 171.196 144.018) (end 171.196 130.967) (width 0.4) (layer "F.Cu") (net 31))
 (segment (start 180.848 110.236) (end 175.006 110.236) (width 0.4) (layer "F.Cu") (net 6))
 (segment (start 186.69 110.236) (end 180.848 110.236) (width 0.4) (layer "F.Cu") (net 6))
 (segment (start 169.413 89.667) (end 177.8 81.28) (width 0.4) (layer "F.Cu") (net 6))
 (segment (start 169.413 94.996) (end 169.413 89.667) (width 0.4) (layer "F.Cu") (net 6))
 (segment (start 175.006 110.236) (end 169.256 110.236) (width 0.4) (layer "F.Cu") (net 6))
 (segment (start 169.256 110.236) (end 169.256 95.153) (width 0.4) (layer "B.Cu") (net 6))
 (segment (start 169.256 95.153) (end 169.413 94.996) (width 0.4) (layer "B.Cu") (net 6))
 (segment (start 169.256 120.396) (end 166.39 117.53) (width 0.4) (layer "B.Cu") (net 25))
 (segment (start 166.39 74.91) (end 175.26 66.04) (width 0.4) (layer "B.Cu") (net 25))
 (segment (start 166.39 117.53) (end 166.39 74.91) (width 0.4) (layer "B.Cu") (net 25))
 (segment (start 173.606 82.201767) (end 174.01 81.797767) (width 0.4) (layer "B.Cu") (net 24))
 (segment (start 173.606 118.996) (end 173.606 82.201767) (width 0.4) (layer "B.Cu") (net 24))
 (segment (start 174.01 81.797767) (end 174.01 69.83) (width 0.4) (layer "B.Cu") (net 24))
 (segment (start 175.006 120.396) (end 173.606 118.996) (width 0.4) (layer "B.Cu") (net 24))
 (segment (start 174.01 69.83) (end 177.8 66.04) (width 0.4) (layer "B.Cu") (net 24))
 (segment (start 176.55 69.83) (end 180.34 66.04) (width 0.4) (layer "B.Cu") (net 23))
 (segment (start 180.848 120.396) (end 176.55 116.098) (width 0.4) (layer "B.Cu") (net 23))
 (segment (start 176.55 116.098) (end 176.55 69.83) (width 0.4) (layer "B.Cu") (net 23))
 (segment (start 185.29 91.483056) (end 179.07 85.263056) (width 0.4) (layer "B.Cu") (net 22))
 (segment (start 179.07 85.263056) (end 179.07 69.85) (width 0.4) (layer "B.Cu") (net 22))
 (segment (start 186.69 120.396) (end 185.29 118.996) (width 0.4) (layer "B.Cu") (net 22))
 (segment (start 185.29 118.996) (end 185.29 91.483056) (width 0.4) (layer "B.Cu") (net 22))
 (segment (start 179.07 69.85) (end 182.88 66.04) (width 0.4) (layer "B.Cu") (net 22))
 (segment (start 192.024 125.984) (end 192.532 125.476) (width 0.4) (layer "F.Cu") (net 7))
 (segment (start 192.024 130.459) (end 192.024 125.984) (width 0.4) (layer "F.Cu") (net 7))
 (segment (start 195.072 99.568) (end 182.88 87.376) (width 0.4) (layer "B.Cu") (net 7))
 (segment (start 182.88 87.376) (end 182.88 81.28) (width 0.4) (layer "B.Cu") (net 7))
 (segment (start 195.072 122.936) (end 195.072 99.568) (width 0.4) (layer "B.Cu") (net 7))
 (segment (start 192.532 125.476) (end 195.072 122.936) (width 0.4) (layer "B.Cu") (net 7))
 (segment (start 192.532 120.396) (end 188.09 115.954) (width 0.4) (layer "B.Cu") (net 21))
 (segment (start 181.61 69.85) (end 185.42 66.04) (width 0.4) (layer "B.Cu") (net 21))
 (segment (start 188.09 93.434528) (end 181.61 86.954528) (width 0.4) (layer "B.Cu") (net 21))
 (segment (start 181.61 86.954528) (end 181.61 69.85) (width 0.4) (layer "B.Cu") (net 21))
 (segment (start 188.09 115.954) (end 188.09 93.434528) (width 0.4) (layer "B.Cu") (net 21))
 (segment (start 174.244 130.459) (end 174.244 126.238) (width 0.4) (layer "F.Cu") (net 35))
 (segment (start 174.244 126.238) (end 175.006 125.476) (width 0.4) (layer "F.Cu") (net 35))
 (segment (start 180.848 126.395) (end 180.848 125.476) (width 0.4) (layer "F.Cu") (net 29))
 (segment (start 176.784 130.459) (end 180.848 126.395) (width 0.4) (layer "F.Cu") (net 29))
 (segment (start 181.707 130.459) (end 186.69 125.476) (width 0.4) (layer "F.Cu") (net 33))
 (segment (start 179.324 130.459) (end 181.707 130.459) (width 0.4) (layer "F.Cu") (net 33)))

